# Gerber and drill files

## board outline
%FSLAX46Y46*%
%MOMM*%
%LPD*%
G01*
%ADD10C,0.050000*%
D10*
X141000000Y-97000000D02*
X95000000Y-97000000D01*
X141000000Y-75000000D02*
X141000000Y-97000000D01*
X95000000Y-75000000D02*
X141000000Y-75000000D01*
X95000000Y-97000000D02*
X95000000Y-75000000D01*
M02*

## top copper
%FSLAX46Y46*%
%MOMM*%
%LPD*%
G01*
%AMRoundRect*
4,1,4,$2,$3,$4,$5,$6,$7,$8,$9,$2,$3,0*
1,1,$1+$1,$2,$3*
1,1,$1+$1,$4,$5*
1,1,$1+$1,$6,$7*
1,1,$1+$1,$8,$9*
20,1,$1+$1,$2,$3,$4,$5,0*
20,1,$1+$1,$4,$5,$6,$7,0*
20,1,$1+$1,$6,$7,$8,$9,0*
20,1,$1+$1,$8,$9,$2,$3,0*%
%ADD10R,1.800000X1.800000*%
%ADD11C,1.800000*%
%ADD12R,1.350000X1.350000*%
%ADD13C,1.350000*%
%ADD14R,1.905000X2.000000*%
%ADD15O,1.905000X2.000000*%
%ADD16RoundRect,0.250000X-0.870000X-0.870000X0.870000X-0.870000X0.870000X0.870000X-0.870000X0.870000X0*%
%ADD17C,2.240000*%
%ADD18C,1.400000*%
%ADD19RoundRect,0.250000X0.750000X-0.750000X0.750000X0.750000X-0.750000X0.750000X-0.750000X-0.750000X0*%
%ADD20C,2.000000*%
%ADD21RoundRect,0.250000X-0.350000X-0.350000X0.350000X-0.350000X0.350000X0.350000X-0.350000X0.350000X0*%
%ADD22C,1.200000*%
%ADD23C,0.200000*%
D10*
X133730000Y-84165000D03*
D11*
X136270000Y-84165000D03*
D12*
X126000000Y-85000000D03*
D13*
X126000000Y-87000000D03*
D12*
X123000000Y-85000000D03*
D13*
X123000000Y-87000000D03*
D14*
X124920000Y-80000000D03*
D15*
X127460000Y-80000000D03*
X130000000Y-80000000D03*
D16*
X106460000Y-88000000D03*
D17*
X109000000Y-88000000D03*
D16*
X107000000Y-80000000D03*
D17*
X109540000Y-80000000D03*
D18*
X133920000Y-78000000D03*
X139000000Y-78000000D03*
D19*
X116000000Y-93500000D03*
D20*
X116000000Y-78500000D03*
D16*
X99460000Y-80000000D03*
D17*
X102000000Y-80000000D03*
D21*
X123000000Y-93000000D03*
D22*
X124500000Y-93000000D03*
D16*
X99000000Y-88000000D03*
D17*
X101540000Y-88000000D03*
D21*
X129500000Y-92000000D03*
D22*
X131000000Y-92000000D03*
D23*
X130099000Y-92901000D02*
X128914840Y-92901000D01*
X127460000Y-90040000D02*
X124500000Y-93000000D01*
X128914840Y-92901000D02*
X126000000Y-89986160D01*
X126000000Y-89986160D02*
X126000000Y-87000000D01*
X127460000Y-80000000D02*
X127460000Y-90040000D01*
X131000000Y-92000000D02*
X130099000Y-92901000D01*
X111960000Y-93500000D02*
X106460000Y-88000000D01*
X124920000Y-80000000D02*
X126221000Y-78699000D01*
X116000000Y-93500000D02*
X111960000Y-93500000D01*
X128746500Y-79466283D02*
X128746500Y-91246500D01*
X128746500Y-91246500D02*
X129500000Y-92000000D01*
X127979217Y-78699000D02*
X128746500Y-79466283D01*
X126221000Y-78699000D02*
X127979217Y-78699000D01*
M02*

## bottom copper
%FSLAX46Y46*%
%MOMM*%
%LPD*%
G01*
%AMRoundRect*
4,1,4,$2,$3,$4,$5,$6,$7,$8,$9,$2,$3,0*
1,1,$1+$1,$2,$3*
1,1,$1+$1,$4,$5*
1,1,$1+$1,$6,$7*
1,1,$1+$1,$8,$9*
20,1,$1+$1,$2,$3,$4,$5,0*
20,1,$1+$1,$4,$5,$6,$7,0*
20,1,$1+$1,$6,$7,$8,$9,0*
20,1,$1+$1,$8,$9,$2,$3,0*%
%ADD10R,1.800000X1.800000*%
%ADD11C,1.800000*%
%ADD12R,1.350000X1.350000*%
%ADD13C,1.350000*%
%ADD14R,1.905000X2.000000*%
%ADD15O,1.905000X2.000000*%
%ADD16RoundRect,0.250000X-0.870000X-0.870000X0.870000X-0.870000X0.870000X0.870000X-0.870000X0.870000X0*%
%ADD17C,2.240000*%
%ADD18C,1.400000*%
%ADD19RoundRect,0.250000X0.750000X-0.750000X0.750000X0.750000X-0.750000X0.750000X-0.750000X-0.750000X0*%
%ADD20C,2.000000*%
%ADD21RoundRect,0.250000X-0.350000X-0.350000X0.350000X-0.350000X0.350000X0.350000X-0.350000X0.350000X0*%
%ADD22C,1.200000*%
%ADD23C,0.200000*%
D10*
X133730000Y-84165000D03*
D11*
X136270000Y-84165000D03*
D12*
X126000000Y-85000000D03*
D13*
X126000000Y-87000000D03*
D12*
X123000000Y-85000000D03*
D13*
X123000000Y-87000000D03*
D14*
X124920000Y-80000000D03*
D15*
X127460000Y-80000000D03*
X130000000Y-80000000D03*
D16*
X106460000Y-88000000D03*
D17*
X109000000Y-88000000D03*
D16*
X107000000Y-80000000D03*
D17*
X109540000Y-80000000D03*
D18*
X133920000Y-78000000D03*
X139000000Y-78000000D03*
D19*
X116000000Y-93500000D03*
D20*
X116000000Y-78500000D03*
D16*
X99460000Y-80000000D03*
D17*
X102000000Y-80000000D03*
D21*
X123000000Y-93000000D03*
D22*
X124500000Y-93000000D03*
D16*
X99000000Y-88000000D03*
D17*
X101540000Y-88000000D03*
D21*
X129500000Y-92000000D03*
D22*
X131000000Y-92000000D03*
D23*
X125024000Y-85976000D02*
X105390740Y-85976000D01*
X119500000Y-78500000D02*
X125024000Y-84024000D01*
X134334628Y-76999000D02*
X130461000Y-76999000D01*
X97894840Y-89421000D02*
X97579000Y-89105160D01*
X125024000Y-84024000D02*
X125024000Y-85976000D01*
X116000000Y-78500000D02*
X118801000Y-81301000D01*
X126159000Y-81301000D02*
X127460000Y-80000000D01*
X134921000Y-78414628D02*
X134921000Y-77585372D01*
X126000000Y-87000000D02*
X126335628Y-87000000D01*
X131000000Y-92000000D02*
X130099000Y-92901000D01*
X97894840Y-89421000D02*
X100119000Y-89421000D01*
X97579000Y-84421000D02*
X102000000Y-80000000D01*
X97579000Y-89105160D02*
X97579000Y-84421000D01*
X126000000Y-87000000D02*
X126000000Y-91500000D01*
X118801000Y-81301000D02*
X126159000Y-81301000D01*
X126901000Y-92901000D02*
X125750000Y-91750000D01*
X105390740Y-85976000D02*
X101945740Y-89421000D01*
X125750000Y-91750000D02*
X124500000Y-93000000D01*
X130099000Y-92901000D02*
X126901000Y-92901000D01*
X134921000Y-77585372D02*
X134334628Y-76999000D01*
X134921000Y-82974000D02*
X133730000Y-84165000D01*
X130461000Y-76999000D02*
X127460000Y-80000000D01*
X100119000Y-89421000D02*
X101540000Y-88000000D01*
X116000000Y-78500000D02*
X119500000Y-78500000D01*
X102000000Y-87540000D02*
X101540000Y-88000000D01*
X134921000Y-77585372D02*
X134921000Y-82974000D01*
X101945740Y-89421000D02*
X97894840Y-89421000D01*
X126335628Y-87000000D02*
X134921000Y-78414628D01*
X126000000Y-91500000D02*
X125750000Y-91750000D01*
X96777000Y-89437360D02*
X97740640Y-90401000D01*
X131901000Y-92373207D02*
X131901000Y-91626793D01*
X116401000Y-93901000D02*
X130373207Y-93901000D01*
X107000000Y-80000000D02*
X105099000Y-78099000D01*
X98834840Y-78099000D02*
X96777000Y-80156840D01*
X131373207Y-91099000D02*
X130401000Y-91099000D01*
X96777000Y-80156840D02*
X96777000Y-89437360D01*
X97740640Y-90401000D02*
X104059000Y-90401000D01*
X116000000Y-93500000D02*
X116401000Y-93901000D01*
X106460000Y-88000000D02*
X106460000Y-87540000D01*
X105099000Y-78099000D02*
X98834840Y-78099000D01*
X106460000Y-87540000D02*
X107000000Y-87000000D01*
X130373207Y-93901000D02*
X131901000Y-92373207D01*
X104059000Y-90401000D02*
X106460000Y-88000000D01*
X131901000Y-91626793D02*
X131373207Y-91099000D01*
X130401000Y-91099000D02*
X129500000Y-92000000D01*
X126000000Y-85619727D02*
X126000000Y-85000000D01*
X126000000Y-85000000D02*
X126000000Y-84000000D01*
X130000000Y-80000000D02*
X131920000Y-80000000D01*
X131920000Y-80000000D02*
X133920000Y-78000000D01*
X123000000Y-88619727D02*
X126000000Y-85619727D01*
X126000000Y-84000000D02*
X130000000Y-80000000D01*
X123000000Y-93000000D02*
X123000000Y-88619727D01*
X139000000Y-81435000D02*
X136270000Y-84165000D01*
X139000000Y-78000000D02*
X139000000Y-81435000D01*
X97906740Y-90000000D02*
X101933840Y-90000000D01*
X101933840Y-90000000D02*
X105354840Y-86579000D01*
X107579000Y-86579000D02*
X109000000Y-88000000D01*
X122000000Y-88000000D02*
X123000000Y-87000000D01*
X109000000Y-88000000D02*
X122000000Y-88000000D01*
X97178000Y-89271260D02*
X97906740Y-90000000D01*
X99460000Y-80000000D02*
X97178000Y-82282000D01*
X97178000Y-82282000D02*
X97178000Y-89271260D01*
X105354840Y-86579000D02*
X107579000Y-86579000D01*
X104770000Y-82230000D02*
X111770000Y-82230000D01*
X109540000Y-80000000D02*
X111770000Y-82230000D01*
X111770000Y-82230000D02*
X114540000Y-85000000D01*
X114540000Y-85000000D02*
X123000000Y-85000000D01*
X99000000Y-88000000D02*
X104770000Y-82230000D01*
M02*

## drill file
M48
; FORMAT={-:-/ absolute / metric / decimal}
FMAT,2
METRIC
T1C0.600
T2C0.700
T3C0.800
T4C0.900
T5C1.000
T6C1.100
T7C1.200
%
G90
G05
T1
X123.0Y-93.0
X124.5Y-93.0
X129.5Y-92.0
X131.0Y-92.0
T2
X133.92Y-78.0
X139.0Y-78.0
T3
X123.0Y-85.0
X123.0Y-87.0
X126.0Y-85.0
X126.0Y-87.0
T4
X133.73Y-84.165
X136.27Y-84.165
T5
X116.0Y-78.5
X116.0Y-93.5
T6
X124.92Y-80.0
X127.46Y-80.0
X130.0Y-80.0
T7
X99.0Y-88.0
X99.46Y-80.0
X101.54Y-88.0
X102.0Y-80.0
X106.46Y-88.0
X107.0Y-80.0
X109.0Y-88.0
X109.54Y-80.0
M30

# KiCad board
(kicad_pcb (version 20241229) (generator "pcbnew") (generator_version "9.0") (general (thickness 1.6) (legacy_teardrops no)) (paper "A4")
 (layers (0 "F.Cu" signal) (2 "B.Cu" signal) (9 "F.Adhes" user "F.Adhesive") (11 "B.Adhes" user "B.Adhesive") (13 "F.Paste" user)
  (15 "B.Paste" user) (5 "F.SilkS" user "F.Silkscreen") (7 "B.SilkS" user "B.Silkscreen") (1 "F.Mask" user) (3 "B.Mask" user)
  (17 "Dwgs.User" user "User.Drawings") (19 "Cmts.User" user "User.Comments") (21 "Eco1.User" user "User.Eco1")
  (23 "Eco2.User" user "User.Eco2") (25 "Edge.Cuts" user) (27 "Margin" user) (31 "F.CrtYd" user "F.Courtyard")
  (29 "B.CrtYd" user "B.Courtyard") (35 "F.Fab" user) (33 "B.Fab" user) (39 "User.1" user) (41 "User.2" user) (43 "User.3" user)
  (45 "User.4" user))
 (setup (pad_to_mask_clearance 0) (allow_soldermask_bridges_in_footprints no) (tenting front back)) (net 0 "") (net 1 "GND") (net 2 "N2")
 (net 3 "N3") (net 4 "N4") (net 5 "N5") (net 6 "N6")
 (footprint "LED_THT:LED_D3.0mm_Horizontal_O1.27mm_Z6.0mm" (layer "F.Cu") (at 133.73 84.165)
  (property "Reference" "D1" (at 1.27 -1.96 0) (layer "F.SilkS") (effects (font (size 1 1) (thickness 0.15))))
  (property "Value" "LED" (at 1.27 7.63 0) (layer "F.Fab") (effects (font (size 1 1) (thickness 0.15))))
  (pad "1" thru_hole rect (at 0 0) (size 1.8 1.8) (drill 0.9) (layers "*.Cu" "*.Mask") (remove_unused_layers no) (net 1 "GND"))
  (pad "2" thru_hole circle (at 2.54 0) (size 1.8 1.8) (drill 0.9) (layers "*.Cu" "*.Mask") (remove_unused_layers no) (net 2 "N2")))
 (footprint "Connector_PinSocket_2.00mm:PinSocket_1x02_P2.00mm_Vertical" (layer "F.Cu") (at 126 85)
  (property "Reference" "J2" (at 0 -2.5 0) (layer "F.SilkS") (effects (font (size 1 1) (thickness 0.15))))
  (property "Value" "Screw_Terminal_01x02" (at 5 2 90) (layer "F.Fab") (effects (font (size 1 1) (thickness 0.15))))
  (pad "1" thru_hole rect (at 0 0) (size 1.35 1.35) (drill 0.8) (layers "*.Cu" "*.Mask") (remove_unused_layers no) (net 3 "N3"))
  (pad "2" thru_hole circle (at 0 2) (size 1.35 1.35) (drill 0.8) (layers "*.Cu" "*.Mask") (remove_unused_layers no) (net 1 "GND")))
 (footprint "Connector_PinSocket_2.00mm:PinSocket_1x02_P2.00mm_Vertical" (layer "F.Cu") (at 123 85)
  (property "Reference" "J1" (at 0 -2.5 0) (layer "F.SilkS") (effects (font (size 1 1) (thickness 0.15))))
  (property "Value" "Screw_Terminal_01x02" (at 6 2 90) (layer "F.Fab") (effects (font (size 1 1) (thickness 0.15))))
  (pad "1" thru_hole rect (at 0 0) (size 1.35 1.35) (drill 0.8) (layers "*.Cu" "*.Mask") (remove_unused_layers no) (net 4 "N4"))
  (pad "2" thru_hole circle (at 0 2) (size 1.35 1.35) (drill 0.8) (layers "*.Cu" "*.Mask") (remove_unused_layers no) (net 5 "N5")))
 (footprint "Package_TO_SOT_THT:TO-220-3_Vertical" (layer "F.Cu") (at 124.92 80)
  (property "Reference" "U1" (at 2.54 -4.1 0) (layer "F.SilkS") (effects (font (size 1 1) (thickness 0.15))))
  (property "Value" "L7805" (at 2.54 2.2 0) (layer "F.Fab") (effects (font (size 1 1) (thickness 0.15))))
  (pad "1" thru_hole rect (at 0 0) (size 1.905 2) (drill 1.1) (layers "*.Cu" "*.Mask") (remove_unused_layers no) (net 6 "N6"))
  (pad "2" thru_hole oval (at 2.54 0) (size 1.905 2) (drill 1.1) (layers "*.Cu" "*.Mask") (remove_unused_layers no) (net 1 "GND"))
  (pad "3" thru_hole oval (at 5.08 0) (size 1.905 2) (drill 1.1) (layers "*.Cu" "*.Mask") (remove_unused_layers no) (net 3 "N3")))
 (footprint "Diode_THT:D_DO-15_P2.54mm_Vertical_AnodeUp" (layer "F.Cu") (at 106.46 88)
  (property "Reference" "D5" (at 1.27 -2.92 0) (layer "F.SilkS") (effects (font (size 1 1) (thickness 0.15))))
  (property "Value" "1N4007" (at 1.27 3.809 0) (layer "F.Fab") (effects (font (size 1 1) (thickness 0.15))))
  (pad "1" thru_hole roundrect (at 0 0) (size 2.24 2.24) (drill 1.2) (layers "*.Cu" "*.Mask") (remove_unused_layers no)
   (roundrect_rratio 0.111607) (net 6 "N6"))
  (pad "2" thru_hole circle (at 2.54 0) (size 2.24 2.24) (drill 1.2) (layers "*.Cu" "*.Mask") (remove_unused_layers no) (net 5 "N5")))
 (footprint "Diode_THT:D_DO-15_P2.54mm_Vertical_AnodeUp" (layer "F.Cu") (at 107 80)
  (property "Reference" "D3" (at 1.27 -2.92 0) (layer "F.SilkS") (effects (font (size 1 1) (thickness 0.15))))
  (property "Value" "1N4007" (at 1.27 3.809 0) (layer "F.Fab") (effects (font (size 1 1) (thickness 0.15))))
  (pad "1" thru_hole roundrect (at 0 0) (size 2.24 2.24) (drill 1.2) (layers "*.Cu" "*.Mask") (remove_unused_layers no)
   (roundrect_rratio 0.111607) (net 6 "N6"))
  (pad "2" thru_hole circle (at 2.54 0) (size 2.24 2.24) (drill 1.2) (layers "*.Cu" "*.Mask") (remove_unused_layers no) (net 4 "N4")))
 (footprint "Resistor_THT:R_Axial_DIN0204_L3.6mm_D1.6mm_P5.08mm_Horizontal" (layer "F.Cu") (at 133.92 78)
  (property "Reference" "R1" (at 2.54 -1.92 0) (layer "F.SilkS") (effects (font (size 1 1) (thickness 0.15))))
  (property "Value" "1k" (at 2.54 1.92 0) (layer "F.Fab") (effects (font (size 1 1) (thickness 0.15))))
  (pad "1" thru_hole circle (at 0 0) (size 1.4 1.4) (drill 0.7) (layers "*.Cu" "*.Mask") (remove_unused_layers no) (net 3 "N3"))
  (pad "2" thru_hole circle (at 5.08 0) (size 1.4 1.4) (drill 0.7) (layers "*.Cu" "*.Mask") (remove_unused_layers no) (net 2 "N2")))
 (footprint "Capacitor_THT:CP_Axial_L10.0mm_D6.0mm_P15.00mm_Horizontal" (layer "F.Cu") (at 116 93.5 90)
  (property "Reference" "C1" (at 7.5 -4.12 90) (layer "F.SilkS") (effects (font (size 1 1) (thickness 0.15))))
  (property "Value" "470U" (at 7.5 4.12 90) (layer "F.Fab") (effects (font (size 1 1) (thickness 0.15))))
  (pad "1" thru_hole roundrect (at 0 0 90) (size 2 2) (drill 1) (layers "*.Cu" "*.Mask") (remove_unused_layers no) (roundrect_rratio 0.125)
   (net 6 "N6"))
  (pad "2" thru_hole circle (at 15 0 90) (size 2 2) (drill 1) (layers "*.Cu" "*.Mask") (remove_unused_layers no) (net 1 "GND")))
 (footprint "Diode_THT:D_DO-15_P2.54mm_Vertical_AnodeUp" (layer "F.Cu") (at 99.46 80)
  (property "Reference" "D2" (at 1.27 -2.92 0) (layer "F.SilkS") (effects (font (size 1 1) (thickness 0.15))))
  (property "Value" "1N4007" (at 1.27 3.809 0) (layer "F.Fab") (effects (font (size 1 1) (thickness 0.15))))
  (pad "1" thru_hole roundrect (at 0 0) (size 2.24 2.24) (drill 1.2) (layers "*.Cu" "*.Mask") (remove_unused_layers no)
   (roundrect_rratio 0.111607) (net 5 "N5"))
  (pad "2" thru_hole circle (at 2.54 0) (size 2.24 2.24) (drill 1.2) (layers "*.Cu" "*.Mask") (remove_unused_layers no) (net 1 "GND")))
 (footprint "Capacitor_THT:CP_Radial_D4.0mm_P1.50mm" (layer "F.Cu") (at 123 93)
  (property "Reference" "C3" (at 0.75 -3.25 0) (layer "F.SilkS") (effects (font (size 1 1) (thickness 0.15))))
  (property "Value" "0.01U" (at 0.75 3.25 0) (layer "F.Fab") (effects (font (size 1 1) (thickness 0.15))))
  (pad "1" thru_hole roundrect (at 0 0) (size 1.2 1.2) (drill 0.6) (layers "*.Cu" "*.Mask") (remove_unused_layers no)
   (roundrect_rratio 0.208333) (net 3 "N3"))
  (pad "2" thru_hole circle (at 1.5 0) (size 1.2 1.2) (drill 0.6) (layers "*.Cu" "*.Mask") (remove_unused_layers no) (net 1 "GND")))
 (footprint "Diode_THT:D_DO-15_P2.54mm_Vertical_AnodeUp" (layer "F.Cu") (at 99 88)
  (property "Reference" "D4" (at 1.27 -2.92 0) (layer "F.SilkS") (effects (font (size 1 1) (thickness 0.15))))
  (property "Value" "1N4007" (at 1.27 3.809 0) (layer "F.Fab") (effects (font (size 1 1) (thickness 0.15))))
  (pad "1" thru_hole roundrect (at 0 0) (size 2.24 2.24) (drill 1.2) (layers "*.Cu" "*.Mask") (remove_unused_layers no)
   (roundrect_rratio 0.111607) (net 4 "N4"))
  (pad "2" thru_hole circle (at 2.54 0) (size 2.24 2.24) (drill 1.2) (layers "*.Cu" "*.Mask") (remove_unused_layers no) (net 1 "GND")))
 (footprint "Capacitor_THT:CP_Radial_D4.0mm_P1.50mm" (layer "F.Cu") (at 129.5 92)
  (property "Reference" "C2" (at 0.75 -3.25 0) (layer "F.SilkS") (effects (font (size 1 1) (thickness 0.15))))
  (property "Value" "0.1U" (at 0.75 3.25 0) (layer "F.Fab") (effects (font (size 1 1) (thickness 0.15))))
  (pad "1" thru_hole roundrect (at 0 0) (size 1.2 1.2) (drill 0.6) (layers "*.Cu" "*.Mask") (remove_unused_layers no)
   (roundrect_rratio 0.208333) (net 6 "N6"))
  (pad "2" thru_hole circle (at 1.5 0) (size 1.2 1.2) (drill 0.6) (layers "*.Cu" "*.Mask") (remove_unused_layers no) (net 1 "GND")))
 (gr_line (start 141 97) (end 95 97) (stroke (width 0.05) (type default)) (layer "Edge.Cuts"))
 (gr_line (start 141 75) (end 141 97) (stroke (width 0.05) (type default)) (layer "Edge.Cuts"))
 (gr_line (start 95 75) (end 141 75) (stroke (width 0.05) (type default)) (layer "Edge.Cuts"))
 (gr_line (start 95 97) (end 95 75) (stroke (width 0.05) (type default)) (layer "Edge.Cuts"))
 (segment (start 130.099 92.901) (end 128.91484 92.901) (width 0.2) (layer "F.Cu") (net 1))
 (segment (start 127.46 90.04) (end 124.5 93) (width 0.2) (layer "F.Cu") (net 1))
 (segment (start 128.91484 92.901) (end 126 89.98616) (width 0.2) (layer "F.Cu") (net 1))
 (segment (start 126 89.98616) (end 126 87) (width 0.2) (layer "F.Cu") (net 1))
 (segment (start 127.46 80) (end 127.46 90.04) (width 0.2) (layer "F.Cu") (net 1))
 (segment (start 131 92) (end 130.099 92.901) (width 0.2) (layer "F.Cu") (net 1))
 (segment (start 125.024 85.976) (end 105.39074 85.976) (width 0.2) (layer "B.Cu") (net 1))
 (segment (start 119.5 78.5) (end 125.024 84.024) (width 0.2) (layer "B.Cu") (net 1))
 (segment (start 134.334628 76.999) (end 130.461 76.999) (width 0.2) (layer "B.Cu") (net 1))
 (segment (start 97.89484 89.421) (end 97.579 89.10516) (width 0.2) (layer "B.Cu") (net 1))
 (segment (start 125.024 84.024) (end 125.024 85.976) (width 0.2) (layer "B.Cu") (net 1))
 (segment (start 116 78.5) (end 118.801 81.301) (width 0.2) (layer "B.Cu") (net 1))
 (segment (start 126.159 81.301) (end 127.46 80) (width 0.2) (layer "B.Cu") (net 1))
 (segment (start 134.921 78.414628) (end 134.921 77.585372) (width 0.2) (layer "B.Cu") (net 1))
 (segment (start 126 87) (end 126.335628 87) (width 0.2) (layer "B.Cu") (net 1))
 (segment (start 131 92) (end 130.099 92.901) (width 0.2) (layer "B.Cu") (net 1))
 (segment (start 97.89484 89.421) (end 100.119 89.421) (width 0.2) (layer "B.Cu") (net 1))
 (segment (start 97.579 84.421) (end 102 80) (width 0.2) (layer "B.Cu") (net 1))
 (segment (start 97.579 89.10516) (end 97.579 84.421) (width 0.2) (layer "B.Cu") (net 1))
 (segment (start 126 87) (end 126 91.5) (width 0.2) (layer "B.Cu") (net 1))
 (segment (start 118.801 81.301) (end 126.159 81.301) (width 0.2) (layer "B.Cu") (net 1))
 (segment (start 126.901 92.901) (end 125.75 91.75) (width 0.2) (layer "B.Cu") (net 1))
 (segment (start 105.39074 85.976) (end 101.94574 89.421) (width 0.2) (layer "B.Cu") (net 1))
 (segment (start 125.75 91.75) (end 124.5 93) (width 0.2) (layer "B.Cu") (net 1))
 (segment (start 130.099 92.901) (end 126.901 92.901) (width 0.2) (layer "B.Cu") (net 1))
 (segment (start 134.921 77.585372) (end 134.334628 76.999) (width 0.2) (layer "B.Cu") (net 1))
 (segment (start 134.921 82.974) (end 133.73 84.165) (width 0.2) (layer "B.Cu") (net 1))
 (segment (start 130.461 76.999) (end 127.46 80) (width 0.2) (layer "B.Cu") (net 1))
 (segment (start 100.119 89.421) (end 101.54 88) (width 0.2) (layer "B.Cu") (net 1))
 (segment (start 116 78.5) (end 119.5 78.5) (width 0.2) (layer "B.Cu") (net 1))
 (segment (start 102 87.54) (end 101.54 88) (width 0.2) (layer "B.Cu") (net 1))
 (segment (start 134.921 77.585372) (end 134.921 82.974) (width 0.2) (layer "B.Cu") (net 1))
 (segment (start 101.94574 89.421) (end 97.89484 89.421) (width 0.2) (layer "B.Cu") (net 1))
 (segment (start 126.335628 87) (end 134.921 78.414628) (width 0.2) (layer "B.Cu") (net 1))
 (segment (start 126 91.5) (end 125.75 91.75) (width 0.2) (layer "B.Cu") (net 1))
 (segment (start 111.96 93.5) (end 106.46 88) (width 0.2) (layer "F.Cu") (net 6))
 (segment (start 124.92 80) (end 126.221 78.699) (width 0.2) (layer "F.Cu") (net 6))
 (segment (start 116 93.5) (end 111.96 93.5) (width 0.2) (layer "F.Cu") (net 6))
 (segment (start 128.7465 79.466283) (end 128.7465 91.2465) (width 0.2) (layer "F.Cu") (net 6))
 (segment (start 128.7465 91.2465) (end 129.5 92) (width 0.2) (layer "F.Cu") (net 6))
 (segment (start 127.979217 78.699) (end 128.7465 79.466283) (width 0.2) (layer "F.Cu") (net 6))
 (segment (start 126.221 78.699) (end 127.979217 78.699) (width 0.2) (layer "F.Cu") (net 6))
 (segment (start 96.777 89.43736) (end 97.74064 90.401) (width 0.2) (layer "B.Cu") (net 6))
 (segment (start 131.901 92.373207) (end 131.901 91.626793) (width 0.2) (layer "B.Cu") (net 6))
 (segment (start 116.401 93.901) (end 130.373207 93.901) (width 0.2) (layer "B.Cu") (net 6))
 (segment (start 107 80) (end 105.099 78.099) (width 0.2) (layer "B.Cu") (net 6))
 (segment (start 98.83484 78.099) (end 96.777 80.15684) (width 0.2) (layer "B.Cu") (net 6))
 (segment (start 131.373207 91.099) (end 130.401 91.099) (width 0.2) (layer "B.Cu") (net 6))
 (segment (start 96.777 80.15684) (end 96.777 89.43736) (width 0.2) (layer "B.Cu") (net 6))
 (segment (start 97.74064 90.401) (end 104.059 90.401) (width 0.2) (layer "B.Cu") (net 6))
 (segment (start 116 93.5) (end 116.401 93.901) (width 0.2) (layer "B.Cu") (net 6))
 (segment (start 106.46 88) (end 106.46 87.54) (width 0.2) (layer "B.Cu") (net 6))
 (segment (start 105.099 78.099) (end 98.83484 78.099) (width 0.2) (layer "B.Cu") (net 6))
 (segment (start 106.46 87.54) (end 107 87) (width 0.2) (layer "B.Cu") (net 6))
 (segment (start 130.373207 93.901) (end 131.901 92.373207) (width 0.2) (layer "B.Cu") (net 6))
 (segment (start 104.059 90.401) (end 106.46 88) (width 0.2) (layer "B.Cu") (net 6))
 (segment (start 131.901 91.626793) (end 131.373207 91.099) (width 0.2) (layer "B.Cu") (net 6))
 (segment (start 130.401 91.099) (end 129.5 92) (width 0.2) (layer "B.Cu") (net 6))
 (segment (start 126 85.619727) (end 126 85) (width 0.2) (layer "B.Cu") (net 3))
 (segment (start 126 85) (end 126 84) (width 0.2) (layer "B.Cu") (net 3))
 (segment (start 130 80) (end 131.92 80) (width 0.2) (layer "B.Cu") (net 3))
 (segment (start 131.92 80) (end 133.92 78) (width 0.2) (layer "B.Cu") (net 3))
 (segment (start 123 88.619727) (end 126 85.619727) (width 0.2) (layer "B.Cu") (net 3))
 (segment (start 126 84) (end 130 80) (width 0.2) (layer "B.Cu") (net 3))
 (segment (start 123 93) (end 123 88.619727) (width 0.2) (layer "B.Cu") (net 3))
 (segment (start 139 81.435) (end 136.27 84.165) (width 0.2) (layer "B.Cu") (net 2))
 (segment (start 139 78) (end 139 81.435) (width 0.2) (layer "B.Cu") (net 2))
 (segment (start 97.90674 90) (end 101.93384 90) (width 0.2) (layer "B.Cu") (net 5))
 (segment (start 101.93384 90) (end 105.35484 86.579) (width 0.2) (layer "B.Cu") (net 5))
 (segment (start 107.579 86.579) (end 109 88) (width 0.2) (layer "B.Cu") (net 5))
 (segment (start 122 88) (end 123 87) (width 0.2) (layer "B.Cu") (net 5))
 (segment (start 109 88) (end 122 88) (width 0.2) (layer "B.Cu") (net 5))
 (segment (start 97.178 89.27126) (end 97.90674 90) (width 0.2) (layer "B.Cu") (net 5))
 (segment (start 99.46 80) (end 97.178 82.282) (width 0.2) (layer "B.Cu") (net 5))
 (segment (start 97.178 82.282) (end 97.178 89.27126) (width 0.2) (layer "B.Cu") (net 5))
 (segment (start 105.35484 86.579) (end 107.579 86.579) (width 0.2) (layer "B.Cu") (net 5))
 (segment (start 104.77 82.23) (end 111.77 82.23) (width 0.2) (layer "B.Cu") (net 4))
 (segment (start 109.54 80) (end 111.77 82.23) (width 0.2) (layer "B.Cu") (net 4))
 (segment (start 111.77 82.23) (end 114.54 85) (width 0.2) (layer "B.Cu") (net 4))
 (segment (start 114.54 85) (end 123 85) (width 0.2) (layer "B.Cu") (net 4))
 (segment (start 99 88) (end 104.77 82.23) (width 0.2) (layer "B.Cu") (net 4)))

